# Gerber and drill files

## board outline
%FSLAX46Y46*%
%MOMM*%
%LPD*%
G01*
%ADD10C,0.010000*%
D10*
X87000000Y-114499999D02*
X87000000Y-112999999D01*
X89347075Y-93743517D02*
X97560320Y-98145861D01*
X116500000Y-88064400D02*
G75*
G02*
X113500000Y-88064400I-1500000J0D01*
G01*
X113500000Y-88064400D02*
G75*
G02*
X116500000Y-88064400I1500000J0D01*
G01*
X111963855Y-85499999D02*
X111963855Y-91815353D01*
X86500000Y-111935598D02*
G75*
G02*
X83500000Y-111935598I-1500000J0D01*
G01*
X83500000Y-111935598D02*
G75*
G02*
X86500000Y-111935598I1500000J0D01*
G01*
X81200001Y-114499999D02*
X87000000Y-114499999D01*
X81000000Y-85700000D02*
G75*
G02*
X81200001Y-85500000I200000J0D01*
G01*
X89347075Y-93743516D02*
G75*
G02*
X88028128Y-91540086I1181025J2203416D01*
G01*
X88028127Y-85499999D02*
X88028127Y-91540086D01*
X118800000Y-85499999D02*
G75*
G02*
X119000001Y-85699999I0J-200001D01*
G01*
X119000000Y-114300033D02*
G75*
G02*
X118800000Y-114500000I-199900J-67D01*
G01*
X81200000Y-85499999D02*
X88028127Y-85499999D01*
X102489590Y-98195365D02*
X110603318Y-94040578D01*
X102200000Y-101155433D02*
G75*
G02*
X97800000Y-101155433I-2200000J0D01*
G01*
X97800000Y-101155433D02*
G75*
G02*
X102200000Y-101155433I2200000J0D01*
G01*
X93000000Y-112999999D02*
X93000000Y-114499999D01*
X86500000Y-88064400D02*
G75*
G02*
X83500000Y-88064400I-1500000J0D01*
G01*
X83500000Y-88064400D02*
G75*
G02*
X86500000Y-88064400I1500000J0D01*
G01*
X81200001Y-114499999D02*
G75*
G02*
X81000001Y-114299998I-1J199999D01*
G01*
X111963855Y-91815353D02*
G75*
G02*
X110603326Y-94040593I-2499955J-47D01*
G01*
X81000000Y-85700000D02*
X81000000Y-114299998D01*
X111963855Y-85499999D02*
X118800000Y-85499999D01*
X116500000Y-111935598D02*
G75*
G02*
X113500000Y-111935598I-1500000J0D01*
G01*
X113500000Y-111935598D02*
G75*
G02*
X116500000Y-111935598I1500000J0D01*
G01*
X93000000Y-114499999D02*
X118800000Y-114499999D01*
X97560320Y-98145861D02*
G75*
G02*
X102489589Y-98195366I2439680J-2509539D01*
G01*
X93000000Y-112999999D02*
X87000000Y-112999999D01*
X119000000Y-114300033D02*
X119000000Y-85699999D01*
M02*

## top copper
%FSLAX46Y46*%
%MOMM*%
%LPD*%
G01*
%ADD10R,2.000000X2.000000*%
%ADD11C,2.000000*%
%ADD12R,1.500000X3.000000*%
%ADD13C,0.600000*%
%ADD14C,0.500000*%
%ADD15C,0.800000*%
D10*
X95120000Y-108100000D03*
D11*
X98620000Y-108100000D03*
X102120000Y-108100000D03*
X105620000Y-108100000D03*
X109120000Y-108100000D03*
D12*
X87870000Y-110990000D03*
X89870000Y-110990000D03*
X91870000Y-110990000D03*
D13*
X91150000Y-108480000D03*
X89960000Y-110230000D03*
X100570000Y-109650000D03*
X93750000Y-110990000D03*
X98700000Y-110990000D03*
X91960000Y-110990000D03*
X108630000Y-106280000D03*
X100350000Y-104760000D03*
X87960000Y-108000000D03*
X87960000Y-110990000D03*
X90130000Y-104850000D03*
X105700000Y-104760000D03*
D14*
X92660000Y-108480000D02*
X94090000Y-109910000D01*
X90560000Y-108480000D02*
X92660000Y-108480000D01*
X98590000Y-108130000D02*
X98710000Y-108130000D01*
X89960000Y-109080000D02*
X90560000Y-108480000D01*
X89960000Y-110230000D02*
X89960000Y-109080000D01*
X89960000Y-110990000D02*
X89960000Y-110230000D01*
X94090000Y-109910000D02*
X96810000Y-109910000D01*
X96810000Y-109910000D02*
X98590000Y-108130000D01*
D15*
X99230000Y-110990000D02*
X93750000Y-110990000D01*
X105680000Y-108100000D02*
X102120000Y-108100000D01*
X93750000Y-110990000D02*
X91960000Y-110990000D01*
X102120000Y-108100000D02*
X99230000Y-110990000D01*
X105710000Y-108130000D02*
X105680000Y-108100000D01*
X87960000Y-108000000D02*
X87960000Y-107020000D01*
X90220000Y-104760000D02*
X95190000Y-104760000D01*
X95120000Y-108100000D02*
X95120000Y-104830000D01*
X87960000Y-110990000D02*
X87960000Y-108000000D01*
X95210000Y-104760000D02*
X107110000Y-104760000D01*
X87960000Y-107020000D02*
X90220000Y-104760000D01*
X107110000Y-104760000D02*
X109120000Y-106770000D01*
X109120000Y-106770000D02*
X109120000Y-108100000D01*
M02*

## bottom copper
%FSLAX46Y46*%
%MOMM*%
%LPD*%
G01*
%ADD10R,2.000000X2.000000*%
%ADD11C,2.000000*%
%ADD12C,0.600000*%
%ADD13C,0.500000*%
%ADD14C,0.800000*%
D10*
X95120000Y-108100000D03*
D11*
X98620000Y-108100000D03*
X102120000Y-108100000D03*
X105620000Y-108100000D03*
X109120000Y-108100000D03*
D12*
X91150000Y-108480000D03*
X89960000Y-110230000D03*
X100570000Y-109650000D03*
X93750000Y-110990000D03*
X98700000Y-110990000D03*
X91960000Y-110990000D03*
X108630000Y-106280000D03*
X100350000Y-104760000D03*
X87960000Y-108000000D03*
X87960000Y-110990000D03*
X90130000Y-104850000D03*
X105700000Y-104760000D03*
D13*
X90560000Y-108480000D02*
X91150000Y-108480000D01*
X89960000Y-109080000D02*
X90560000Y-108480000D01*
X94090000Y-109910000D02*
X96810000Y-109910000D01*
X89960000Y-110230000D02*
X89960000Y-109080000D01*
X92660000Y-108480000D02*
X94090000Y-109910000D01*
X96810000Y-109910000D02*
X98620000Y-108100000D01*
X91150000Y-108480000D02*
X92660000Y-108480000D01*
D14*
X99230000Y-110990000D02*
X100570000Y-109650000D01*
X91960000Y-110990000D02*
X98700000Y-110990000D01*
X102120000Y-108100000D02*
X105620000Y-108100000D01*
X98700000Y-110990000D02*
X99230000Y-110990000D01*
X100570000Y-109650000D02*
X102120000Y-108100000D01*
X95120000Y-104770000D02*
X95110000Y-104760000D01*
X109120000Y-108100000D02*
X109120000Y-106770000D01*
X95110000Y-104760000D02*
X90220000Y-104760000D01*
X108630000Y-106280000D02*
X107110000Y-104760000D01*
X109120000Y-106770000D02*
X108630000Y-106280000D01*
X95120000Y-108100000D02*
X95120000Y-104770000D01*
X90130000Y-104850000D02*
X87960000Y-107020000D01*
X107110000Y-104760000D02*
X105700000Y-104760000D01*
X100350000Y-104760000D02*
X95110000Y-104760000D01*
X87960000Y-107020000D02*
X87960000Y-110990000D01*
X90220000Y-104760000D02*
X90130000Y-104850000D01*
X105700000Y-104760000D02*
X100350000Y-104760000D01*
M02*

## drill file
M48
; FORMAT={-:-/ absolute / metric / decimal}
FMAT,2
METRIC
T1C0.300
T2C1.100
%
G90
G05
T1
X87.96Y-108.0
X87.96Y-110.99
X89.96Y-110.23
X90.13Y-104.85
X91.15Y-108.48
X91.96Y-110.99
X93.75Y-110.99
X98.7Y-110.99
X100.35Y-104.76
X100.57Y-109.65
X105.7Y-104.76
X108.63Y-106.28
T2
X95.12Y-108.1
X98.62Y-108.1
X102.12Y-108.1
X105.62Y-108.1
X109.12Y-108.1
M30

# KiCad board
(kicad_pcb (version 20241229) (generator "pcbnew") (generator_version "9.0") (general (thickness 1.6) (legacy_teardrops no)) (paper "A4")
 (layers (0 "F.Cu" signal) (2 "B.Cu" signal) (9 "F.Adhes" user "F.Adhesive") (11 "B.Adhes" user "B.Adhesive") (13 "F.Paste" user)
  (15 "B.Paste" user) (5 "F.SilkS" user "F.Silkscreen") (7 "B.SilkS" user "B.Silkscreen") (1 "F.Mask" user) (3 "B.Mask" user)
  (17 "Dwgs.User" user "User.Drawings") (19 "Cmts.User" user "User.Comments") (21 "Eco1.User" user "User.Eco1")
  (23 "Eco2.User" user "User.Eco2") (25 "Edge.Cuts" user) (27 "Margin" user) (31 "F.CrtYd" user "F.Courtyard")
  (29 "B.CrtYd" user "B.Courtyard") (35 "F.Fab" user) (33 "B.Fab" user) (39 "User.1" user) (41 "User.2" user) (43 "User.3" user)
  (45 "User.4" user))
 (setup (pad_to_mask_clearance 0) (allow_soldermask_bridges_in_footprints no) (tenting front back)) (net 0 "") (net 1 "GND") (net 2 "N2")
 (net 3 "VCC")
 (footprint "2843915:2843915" (layer "F.Cu") (at 95.12 108.1)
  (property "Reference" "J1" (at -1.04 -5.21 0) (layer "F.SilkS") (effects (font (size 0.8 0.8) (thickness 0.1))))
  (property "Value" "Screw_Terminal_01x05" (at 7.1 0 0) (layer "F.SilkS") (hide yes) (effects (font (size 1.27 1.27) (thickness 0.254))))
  (pad "1" thru_hole rect (at 0 0) (size 2 2) (drill 1.1) (layers "*.Cu" "*.Mask") (remove_unused_layers no) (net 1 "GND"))
  (pad "2" thru_hole circle (at 3.5 0) (size 2 2) (drill 1.1) (layers "*.Cu" "*.Mask") (remove_unused_layers no) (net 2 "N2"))
  (pad "3" thru_hole circle (at 7 0) (size 2 2) (drill 1.1) (layers "*.Cu" "*.Mask") (remove_unused_layers no) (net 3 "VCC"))
  (pad "4" thru_hole circle (at 10.5 0) (size 2 2) (drill 1.1) (layers "*.Cu" "*.Mask") (remove_unused_layers no) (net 3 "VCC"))
  (pad "5" thru_hole circle (at 14 0) (size 2 2) (drill 1.1) (layers "*.Cu" "*.Mask") (remove_unused_layers no) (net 1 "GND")))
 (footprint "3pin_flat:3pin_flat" (layer "F.Cu") (at 89.87 109.39 180)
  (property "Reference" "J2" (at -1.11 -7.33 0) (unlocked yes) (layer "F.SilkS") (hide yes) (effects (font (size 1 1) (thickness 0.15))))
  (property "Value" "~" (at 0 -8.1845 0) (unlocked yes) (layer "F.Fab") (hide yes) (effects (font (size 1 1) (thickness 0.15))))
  (pad "1" smd rect (at 2 -1.6 180) (size 1.5 3) (layers "F.Cu" "F.Mask" "F.Paste") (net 1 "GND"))
  (pad "2" smd rect (at 0 -1.6 180) (size 1.5 3) (layers "F.Cu" "F.Mask" "F.Paste") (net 2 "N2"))
  (pad "3" smd rect (at -2 -1.6 180) (size 1.5 3) (layers "F.Cu" "F.Mask" "F.Paste") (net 3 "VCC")))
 (gr_line (start 87 114.499999) (end 87 112.999999) (stroke (width 0.01) (type default)) (layer "Edge.Cuts"))
 (gr_line (start 89.347075 93.743517) (end 97.56032 98.145861) (stroke (width 0.01) (type default)) (layer "Edge.Cuts"))
 (gr_circle (center 115 88.0644) (end 116.5 88.0644) (stroke (width 0.01) (type default)) (fill no) (layer "Edge.Cuts"))
 (gr_line (start 111.963855 85.499999) (end 111.963855 91.815353) (stroke (width 0.01) (type default)) (layer "Edge.Cuts"))
 (gr_circle (center 85 111.935598) (end 86.5 111.935598) (stroke (width 0.01) (type default)) (fill no) (layer "Edge.Cuts"))
 (gr_line (start 81.200001 114.499999) (end 87 114.499999) (stroke (width 0.01) (type default)) (layer "Edge.Cuts"))
 (gr_arc (start 81 85.7) (mid 81.058579 85.558578) (end 81.200001 85.499999) (stroke (width 0.01) (type default)) (layer "Edge.Cuts"))
 (gr_arc (start 89.347075 93.743516) (mid 88.383059 92.824095) (end 88.028127 91.540086) (stroke (width 0.01) (type default))
  (layer "Edge.Cuts"))
 (gr_line (start 88.028127 85.499999) (end 88.028127 91.540086) (stroke (width 0.01) (type default)) (layer "Edge.Cuts"))
 (gr_arc (start 118.8 85.499999) (mid 118.941433 85.558576) (end 119 85.699999) (stroke (width 0.01) (type default)) (layer "Edge.Cuts"))
 (gr_arc (start 119 114.300033) (mid 118.941433 114.441442) (end 118.8 114.499999) (stroke (width 0.01) (type default)) (layer "Edge.Cuts"))
 (gr_line (start 81.2 85.499999) (end 88.028127 85.499999) (stroke (width 0.01) (type default)) (layer "Edge.Cuts"))
 (gr_line (start 102.48959 98.195365) (end 110.603318 94.040578) (stroke (width 0.01) (type default)) (layer "Edge.Cuts"))
 (gr_circle (center 100 101.155433) (end 102.2 101.155433) (stroke (width 0.01) (type default)) (fill no) (layer "Edge.Cuts"))
 (gr_line (start 93 112.999999) (end 93 114.499999) (stroke (width 0.01) (type default)) (layer "Edge.Cuts"))
 (gr_circle (center 85 88.0644) (end 86.5 88.0644) (stroke (width 0.01) (type default)) (fill no) (layer "Edge.Cuts"))
 (gr_arc (start 81.200001 114.499999) (mid 81.058579 114.44142) (end 81 114.299998) (stroke (width 0.01) (type default)) (layer "Edge.Cuts"))
 (gr_arc (start 111.963855 91.815353) (mid 111.596771 93.119449) (end 110.603318 94.040578) (stroke (width 0.01) (type default))
  (layer "Edge.Cuts"))
 (gr_line (start 81 85.7) (end 81 114.299998) (stroke (width 0.01) (type default)) (layer "Edge.Cuts"))
 (gr_line (start 111.963855 85.499999) (end 118.8 85.499999) (stroke (width 0.01) (type solid)) (layer "Edge.Cuts"))
 (gr_circle (center 115 111.935598) (end 116.5 111.935598) (stroke (width 0.01) (type default)) (fill no) (layer "Edge.Cuts"))
 (gr_line (start 93 114.499999) (end 118.8 114.499999) (stroke (width 0.01) (type default)) (layer "Edge.Cuts"))
 (gr_arc (start 97.56032 98.145861) (mid 100.035149 97.155609) (end 102.48959 98.195365) (stroke (width 0.01) (type default))
  (layer "Edge.Cuts"))
 (gr_line (start 93 112.999999) (end 87 112.999999) (stroke (width 0.01) (type default)) (layer "Edge.Cuts"))
 (gr_line (start 119 114.300033) (end 119 85.699999) (stroke (width 0.01) (type default)) (layer "Edge.Cuts"))
 (segment (start 92.66 108.48) (end 94.09 109.91) (width 0.5) (layer "F.Cu") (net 2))
 (segment (start 90.56 108.48) (end 92.66 108.48) (width 0.5) (layer "F.Cu") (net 2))
 (segment (start 98.59 108.13) (end 98.71 108.13) (width 0.5) (layer "F.Cu") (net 2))
 (segment (start 89.96 109.08) (end 90.56 108.48) (width 0.5) (layer "F.Cu") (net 2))
 (segment (start 89.96 110.23) (end 89.96 109.08) (width 0.5) (layer "F.Cu") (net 2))
 (segment (start 89.96 110.99) (end 89.96 110.23) (width 0.5) (layer "F.Cu") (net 2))
 (segment (start 94.09 109.91) (end 96.81 109.91) (width 0.5) (layer "F.Cu") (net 2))
 (segment (start 96.81 109.91) (end 98.59 108.13) (width 0.5) (layer "F.Cu") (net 2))
 (via (at 91.15 108.48) (size 0.6) (drill 0.3) (layers "F.Cu" "B.Cu") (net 2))
 (via (at 89.96 110.23) (size 0.6) (drill 0.3) (layers "F.Cu" "B.Cu") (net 2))
 (segment (start 90.56 108.48) (end 91.15 108.48) (width 0.5) (layer "B.Cu") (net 2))
 (segment (start 89.96 109.08) (end 90.56 108.48) (width 0.5) (layer "B.Cu") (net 2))
 (segment (start 94.09 109.91) (end 96.81 109.91) (width 0.5) (layer "B.Cu") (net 2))
 (segment (start 89.96 110.23) (end 89.96 109.08) (width 0.5) (layer "B.Cu") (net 2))
 (segment (start 92.66 108.48) (end 94.09 109.91) (width 0.5) (layer "B.Cu") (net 2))
 (segment (start 96.81 109.91) (end 98.62 108.1) (width 0.5) (layer "B.Cu") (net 2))
 (segment (start 91.15 108.48) (end 92.66 108.48) (width 0.5) (layer "B.Cu") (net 2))
 (segment (start 99.23 110.99) (end 93.75 110.99) (width 0.8) (layer "F.Cu") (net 3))
 (segment (start 105.68 108.1) (end 102.12 108.1) (width 0.8) (layer "F.Cu") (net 3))
 (segment (start 93.75 110.99) (end 91.96 110.99) (width 0.8) (layer "F.Cu") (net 3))
 (segment (start 102.12 108.1) (end 99.23 110.99) (width 0.8) (layer "F.Cu") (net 3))
 (segment (start 105.71 108.13) (end 105.68 108.1) (width 0.8) (layer "F.Cu") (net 3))
 (via (at 100.57 109.65) (size 0.6) (drill 0.3) (layers "F.Cu" "B.Cu") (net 3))
 (via (at 93.75 110.99) (size 0.6) (drill 0.3) (layers "F.Cu" "B.Cu") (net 3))
 (via (at 98.7 110.99) (size 0.6) (drill 0.3) (layers "F.Cu" "B.Cu") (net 3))
 (via (at 91.96 110.99) (size 0.6) (drill 0.3) (layers "F.Cu" "B.Cu") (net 3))
 (segment (start 99.23 110.99) (end 100.57 109.65) (width 0.8) (layer "B.Cu") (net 3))
 (segment (start 91.96 110.99) (end 98.7 110.99) (width 0.8) (layer "B.Cu") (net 3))
 (segment (start 102.12 108.1) (end 105.62 108.1) (width 0.8) (layer "B.Cu") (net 3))
 (segment (start 98.7 110.99) (end 99.23 110.99) (width 0.8) (layer "B.Cu") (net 3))
 (segment (start 100.57 109.65) (end 102.12 108.1) (width 0.8) (layer "B.Cu") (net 3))
 (segment (start 87.96 108) (end 87.96 107.02) (width 0.8) (layer "F.Cu") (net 1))
 (segment (start 90.22 104.76) (end 95.19 104.76) (width 0.8) (layer "F.Cu") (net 1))
 (segment (start 95.12 108.1) (end 95.12 104.83) (width 0.8) (layer "F.Cu") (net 1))
 (segment (start 87.96 110.99) (end 87.96 108) (width 0.8) (layer "F.Cu") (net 1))
 (segment (start 95.21 104.76) (end 107.11 104.76) (width 0.8) (layer "F.Cu") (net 1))
 (segment (start 87.96 107.02) (end 90.22 104.76) (width 0.8) (layer "F.Cu") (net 1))
 (segment (start 107.11 104.76) (end 109.12 106.77) (width 0.8) (layer "F.Cu") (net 1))
 (segment (start 109.12 106.77) (end 109.12 108.1) (width 0.8) (layer "F.Cu") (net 1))
 (via (at 108.63 106.28) (size 0.6) (drill 0.3) (layers "F.Cu" "B.Cu") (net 1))
 (via (at 100.35 104.76) (size 0.6) (drill 0.3) (layers "F.Cu" "B.Cu") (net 1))
 (via (at 87.96 108) (size 0.6) (drill 0.3) (layers "F.Cu" "B.Cu") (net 1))
 (via (at 87.96 110.99) (size 0.6) (drill 0.3) (layers "F.Cu" "B.Cu") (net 1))
 (via (at 90.13 104.85) (size 0.6) (drill 0.3) (layers "F.Cu" "B.Cu") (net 1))
 (via (at 105.7 104.76) (size 0.6) (drill 0.3) (layers "F.Cu" "B.Cu") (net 1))
 (segment (start 95.12 104.77) (end 95.11 104.76) (width 0.8) (layer "B.Cu") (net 1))
 (segment (start 109.12 108.1) (end 109.12 106.77) (width 0.8) (layer "B.Cu") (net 1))
 (segment (start 95.11 104.76) (end 90.22 104.76) (width 0.8) (layer "B.Cu") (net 1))
 (segment (start 108.63 106.28) (end 107.11 104.76) (width 0.8) (layer "B.Cu") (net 1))
 (segment (start 109.12 106.77) (end 108.63 106.28) (width 0.8) (layer "B.Cu") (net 1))
 (segment (start 95.12 108.1) (end 95.12 104.77) (width 0.8) (layer "B.Cu") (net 1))
 (segment (start 90.13 104.85) (end 87.96 107.02) (width 0.8) (layer "B.Cu") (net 1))
 (segment (start 107.11 104.76) (end 105.7 104.76) (width 0.8) (layer "B.Cu") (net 1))
 (segment (start 100.35 104.76) (end 95.11 104.76) (width 0.8) (layer "B.Cu") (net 1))
 (segment (start 87.96 107.02) (end 87.96 110.99) (width 0.8) (layer "B.Cu") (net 1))
 (segment (start 90.22 104.76) (end 90.13 104.85) (width 0.8) (layer "B.Cu") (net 1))
 (segment (start 105.7 104.76) (end 100.35 104.76) (width 0.8) (layer "B.Cu") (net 1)))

